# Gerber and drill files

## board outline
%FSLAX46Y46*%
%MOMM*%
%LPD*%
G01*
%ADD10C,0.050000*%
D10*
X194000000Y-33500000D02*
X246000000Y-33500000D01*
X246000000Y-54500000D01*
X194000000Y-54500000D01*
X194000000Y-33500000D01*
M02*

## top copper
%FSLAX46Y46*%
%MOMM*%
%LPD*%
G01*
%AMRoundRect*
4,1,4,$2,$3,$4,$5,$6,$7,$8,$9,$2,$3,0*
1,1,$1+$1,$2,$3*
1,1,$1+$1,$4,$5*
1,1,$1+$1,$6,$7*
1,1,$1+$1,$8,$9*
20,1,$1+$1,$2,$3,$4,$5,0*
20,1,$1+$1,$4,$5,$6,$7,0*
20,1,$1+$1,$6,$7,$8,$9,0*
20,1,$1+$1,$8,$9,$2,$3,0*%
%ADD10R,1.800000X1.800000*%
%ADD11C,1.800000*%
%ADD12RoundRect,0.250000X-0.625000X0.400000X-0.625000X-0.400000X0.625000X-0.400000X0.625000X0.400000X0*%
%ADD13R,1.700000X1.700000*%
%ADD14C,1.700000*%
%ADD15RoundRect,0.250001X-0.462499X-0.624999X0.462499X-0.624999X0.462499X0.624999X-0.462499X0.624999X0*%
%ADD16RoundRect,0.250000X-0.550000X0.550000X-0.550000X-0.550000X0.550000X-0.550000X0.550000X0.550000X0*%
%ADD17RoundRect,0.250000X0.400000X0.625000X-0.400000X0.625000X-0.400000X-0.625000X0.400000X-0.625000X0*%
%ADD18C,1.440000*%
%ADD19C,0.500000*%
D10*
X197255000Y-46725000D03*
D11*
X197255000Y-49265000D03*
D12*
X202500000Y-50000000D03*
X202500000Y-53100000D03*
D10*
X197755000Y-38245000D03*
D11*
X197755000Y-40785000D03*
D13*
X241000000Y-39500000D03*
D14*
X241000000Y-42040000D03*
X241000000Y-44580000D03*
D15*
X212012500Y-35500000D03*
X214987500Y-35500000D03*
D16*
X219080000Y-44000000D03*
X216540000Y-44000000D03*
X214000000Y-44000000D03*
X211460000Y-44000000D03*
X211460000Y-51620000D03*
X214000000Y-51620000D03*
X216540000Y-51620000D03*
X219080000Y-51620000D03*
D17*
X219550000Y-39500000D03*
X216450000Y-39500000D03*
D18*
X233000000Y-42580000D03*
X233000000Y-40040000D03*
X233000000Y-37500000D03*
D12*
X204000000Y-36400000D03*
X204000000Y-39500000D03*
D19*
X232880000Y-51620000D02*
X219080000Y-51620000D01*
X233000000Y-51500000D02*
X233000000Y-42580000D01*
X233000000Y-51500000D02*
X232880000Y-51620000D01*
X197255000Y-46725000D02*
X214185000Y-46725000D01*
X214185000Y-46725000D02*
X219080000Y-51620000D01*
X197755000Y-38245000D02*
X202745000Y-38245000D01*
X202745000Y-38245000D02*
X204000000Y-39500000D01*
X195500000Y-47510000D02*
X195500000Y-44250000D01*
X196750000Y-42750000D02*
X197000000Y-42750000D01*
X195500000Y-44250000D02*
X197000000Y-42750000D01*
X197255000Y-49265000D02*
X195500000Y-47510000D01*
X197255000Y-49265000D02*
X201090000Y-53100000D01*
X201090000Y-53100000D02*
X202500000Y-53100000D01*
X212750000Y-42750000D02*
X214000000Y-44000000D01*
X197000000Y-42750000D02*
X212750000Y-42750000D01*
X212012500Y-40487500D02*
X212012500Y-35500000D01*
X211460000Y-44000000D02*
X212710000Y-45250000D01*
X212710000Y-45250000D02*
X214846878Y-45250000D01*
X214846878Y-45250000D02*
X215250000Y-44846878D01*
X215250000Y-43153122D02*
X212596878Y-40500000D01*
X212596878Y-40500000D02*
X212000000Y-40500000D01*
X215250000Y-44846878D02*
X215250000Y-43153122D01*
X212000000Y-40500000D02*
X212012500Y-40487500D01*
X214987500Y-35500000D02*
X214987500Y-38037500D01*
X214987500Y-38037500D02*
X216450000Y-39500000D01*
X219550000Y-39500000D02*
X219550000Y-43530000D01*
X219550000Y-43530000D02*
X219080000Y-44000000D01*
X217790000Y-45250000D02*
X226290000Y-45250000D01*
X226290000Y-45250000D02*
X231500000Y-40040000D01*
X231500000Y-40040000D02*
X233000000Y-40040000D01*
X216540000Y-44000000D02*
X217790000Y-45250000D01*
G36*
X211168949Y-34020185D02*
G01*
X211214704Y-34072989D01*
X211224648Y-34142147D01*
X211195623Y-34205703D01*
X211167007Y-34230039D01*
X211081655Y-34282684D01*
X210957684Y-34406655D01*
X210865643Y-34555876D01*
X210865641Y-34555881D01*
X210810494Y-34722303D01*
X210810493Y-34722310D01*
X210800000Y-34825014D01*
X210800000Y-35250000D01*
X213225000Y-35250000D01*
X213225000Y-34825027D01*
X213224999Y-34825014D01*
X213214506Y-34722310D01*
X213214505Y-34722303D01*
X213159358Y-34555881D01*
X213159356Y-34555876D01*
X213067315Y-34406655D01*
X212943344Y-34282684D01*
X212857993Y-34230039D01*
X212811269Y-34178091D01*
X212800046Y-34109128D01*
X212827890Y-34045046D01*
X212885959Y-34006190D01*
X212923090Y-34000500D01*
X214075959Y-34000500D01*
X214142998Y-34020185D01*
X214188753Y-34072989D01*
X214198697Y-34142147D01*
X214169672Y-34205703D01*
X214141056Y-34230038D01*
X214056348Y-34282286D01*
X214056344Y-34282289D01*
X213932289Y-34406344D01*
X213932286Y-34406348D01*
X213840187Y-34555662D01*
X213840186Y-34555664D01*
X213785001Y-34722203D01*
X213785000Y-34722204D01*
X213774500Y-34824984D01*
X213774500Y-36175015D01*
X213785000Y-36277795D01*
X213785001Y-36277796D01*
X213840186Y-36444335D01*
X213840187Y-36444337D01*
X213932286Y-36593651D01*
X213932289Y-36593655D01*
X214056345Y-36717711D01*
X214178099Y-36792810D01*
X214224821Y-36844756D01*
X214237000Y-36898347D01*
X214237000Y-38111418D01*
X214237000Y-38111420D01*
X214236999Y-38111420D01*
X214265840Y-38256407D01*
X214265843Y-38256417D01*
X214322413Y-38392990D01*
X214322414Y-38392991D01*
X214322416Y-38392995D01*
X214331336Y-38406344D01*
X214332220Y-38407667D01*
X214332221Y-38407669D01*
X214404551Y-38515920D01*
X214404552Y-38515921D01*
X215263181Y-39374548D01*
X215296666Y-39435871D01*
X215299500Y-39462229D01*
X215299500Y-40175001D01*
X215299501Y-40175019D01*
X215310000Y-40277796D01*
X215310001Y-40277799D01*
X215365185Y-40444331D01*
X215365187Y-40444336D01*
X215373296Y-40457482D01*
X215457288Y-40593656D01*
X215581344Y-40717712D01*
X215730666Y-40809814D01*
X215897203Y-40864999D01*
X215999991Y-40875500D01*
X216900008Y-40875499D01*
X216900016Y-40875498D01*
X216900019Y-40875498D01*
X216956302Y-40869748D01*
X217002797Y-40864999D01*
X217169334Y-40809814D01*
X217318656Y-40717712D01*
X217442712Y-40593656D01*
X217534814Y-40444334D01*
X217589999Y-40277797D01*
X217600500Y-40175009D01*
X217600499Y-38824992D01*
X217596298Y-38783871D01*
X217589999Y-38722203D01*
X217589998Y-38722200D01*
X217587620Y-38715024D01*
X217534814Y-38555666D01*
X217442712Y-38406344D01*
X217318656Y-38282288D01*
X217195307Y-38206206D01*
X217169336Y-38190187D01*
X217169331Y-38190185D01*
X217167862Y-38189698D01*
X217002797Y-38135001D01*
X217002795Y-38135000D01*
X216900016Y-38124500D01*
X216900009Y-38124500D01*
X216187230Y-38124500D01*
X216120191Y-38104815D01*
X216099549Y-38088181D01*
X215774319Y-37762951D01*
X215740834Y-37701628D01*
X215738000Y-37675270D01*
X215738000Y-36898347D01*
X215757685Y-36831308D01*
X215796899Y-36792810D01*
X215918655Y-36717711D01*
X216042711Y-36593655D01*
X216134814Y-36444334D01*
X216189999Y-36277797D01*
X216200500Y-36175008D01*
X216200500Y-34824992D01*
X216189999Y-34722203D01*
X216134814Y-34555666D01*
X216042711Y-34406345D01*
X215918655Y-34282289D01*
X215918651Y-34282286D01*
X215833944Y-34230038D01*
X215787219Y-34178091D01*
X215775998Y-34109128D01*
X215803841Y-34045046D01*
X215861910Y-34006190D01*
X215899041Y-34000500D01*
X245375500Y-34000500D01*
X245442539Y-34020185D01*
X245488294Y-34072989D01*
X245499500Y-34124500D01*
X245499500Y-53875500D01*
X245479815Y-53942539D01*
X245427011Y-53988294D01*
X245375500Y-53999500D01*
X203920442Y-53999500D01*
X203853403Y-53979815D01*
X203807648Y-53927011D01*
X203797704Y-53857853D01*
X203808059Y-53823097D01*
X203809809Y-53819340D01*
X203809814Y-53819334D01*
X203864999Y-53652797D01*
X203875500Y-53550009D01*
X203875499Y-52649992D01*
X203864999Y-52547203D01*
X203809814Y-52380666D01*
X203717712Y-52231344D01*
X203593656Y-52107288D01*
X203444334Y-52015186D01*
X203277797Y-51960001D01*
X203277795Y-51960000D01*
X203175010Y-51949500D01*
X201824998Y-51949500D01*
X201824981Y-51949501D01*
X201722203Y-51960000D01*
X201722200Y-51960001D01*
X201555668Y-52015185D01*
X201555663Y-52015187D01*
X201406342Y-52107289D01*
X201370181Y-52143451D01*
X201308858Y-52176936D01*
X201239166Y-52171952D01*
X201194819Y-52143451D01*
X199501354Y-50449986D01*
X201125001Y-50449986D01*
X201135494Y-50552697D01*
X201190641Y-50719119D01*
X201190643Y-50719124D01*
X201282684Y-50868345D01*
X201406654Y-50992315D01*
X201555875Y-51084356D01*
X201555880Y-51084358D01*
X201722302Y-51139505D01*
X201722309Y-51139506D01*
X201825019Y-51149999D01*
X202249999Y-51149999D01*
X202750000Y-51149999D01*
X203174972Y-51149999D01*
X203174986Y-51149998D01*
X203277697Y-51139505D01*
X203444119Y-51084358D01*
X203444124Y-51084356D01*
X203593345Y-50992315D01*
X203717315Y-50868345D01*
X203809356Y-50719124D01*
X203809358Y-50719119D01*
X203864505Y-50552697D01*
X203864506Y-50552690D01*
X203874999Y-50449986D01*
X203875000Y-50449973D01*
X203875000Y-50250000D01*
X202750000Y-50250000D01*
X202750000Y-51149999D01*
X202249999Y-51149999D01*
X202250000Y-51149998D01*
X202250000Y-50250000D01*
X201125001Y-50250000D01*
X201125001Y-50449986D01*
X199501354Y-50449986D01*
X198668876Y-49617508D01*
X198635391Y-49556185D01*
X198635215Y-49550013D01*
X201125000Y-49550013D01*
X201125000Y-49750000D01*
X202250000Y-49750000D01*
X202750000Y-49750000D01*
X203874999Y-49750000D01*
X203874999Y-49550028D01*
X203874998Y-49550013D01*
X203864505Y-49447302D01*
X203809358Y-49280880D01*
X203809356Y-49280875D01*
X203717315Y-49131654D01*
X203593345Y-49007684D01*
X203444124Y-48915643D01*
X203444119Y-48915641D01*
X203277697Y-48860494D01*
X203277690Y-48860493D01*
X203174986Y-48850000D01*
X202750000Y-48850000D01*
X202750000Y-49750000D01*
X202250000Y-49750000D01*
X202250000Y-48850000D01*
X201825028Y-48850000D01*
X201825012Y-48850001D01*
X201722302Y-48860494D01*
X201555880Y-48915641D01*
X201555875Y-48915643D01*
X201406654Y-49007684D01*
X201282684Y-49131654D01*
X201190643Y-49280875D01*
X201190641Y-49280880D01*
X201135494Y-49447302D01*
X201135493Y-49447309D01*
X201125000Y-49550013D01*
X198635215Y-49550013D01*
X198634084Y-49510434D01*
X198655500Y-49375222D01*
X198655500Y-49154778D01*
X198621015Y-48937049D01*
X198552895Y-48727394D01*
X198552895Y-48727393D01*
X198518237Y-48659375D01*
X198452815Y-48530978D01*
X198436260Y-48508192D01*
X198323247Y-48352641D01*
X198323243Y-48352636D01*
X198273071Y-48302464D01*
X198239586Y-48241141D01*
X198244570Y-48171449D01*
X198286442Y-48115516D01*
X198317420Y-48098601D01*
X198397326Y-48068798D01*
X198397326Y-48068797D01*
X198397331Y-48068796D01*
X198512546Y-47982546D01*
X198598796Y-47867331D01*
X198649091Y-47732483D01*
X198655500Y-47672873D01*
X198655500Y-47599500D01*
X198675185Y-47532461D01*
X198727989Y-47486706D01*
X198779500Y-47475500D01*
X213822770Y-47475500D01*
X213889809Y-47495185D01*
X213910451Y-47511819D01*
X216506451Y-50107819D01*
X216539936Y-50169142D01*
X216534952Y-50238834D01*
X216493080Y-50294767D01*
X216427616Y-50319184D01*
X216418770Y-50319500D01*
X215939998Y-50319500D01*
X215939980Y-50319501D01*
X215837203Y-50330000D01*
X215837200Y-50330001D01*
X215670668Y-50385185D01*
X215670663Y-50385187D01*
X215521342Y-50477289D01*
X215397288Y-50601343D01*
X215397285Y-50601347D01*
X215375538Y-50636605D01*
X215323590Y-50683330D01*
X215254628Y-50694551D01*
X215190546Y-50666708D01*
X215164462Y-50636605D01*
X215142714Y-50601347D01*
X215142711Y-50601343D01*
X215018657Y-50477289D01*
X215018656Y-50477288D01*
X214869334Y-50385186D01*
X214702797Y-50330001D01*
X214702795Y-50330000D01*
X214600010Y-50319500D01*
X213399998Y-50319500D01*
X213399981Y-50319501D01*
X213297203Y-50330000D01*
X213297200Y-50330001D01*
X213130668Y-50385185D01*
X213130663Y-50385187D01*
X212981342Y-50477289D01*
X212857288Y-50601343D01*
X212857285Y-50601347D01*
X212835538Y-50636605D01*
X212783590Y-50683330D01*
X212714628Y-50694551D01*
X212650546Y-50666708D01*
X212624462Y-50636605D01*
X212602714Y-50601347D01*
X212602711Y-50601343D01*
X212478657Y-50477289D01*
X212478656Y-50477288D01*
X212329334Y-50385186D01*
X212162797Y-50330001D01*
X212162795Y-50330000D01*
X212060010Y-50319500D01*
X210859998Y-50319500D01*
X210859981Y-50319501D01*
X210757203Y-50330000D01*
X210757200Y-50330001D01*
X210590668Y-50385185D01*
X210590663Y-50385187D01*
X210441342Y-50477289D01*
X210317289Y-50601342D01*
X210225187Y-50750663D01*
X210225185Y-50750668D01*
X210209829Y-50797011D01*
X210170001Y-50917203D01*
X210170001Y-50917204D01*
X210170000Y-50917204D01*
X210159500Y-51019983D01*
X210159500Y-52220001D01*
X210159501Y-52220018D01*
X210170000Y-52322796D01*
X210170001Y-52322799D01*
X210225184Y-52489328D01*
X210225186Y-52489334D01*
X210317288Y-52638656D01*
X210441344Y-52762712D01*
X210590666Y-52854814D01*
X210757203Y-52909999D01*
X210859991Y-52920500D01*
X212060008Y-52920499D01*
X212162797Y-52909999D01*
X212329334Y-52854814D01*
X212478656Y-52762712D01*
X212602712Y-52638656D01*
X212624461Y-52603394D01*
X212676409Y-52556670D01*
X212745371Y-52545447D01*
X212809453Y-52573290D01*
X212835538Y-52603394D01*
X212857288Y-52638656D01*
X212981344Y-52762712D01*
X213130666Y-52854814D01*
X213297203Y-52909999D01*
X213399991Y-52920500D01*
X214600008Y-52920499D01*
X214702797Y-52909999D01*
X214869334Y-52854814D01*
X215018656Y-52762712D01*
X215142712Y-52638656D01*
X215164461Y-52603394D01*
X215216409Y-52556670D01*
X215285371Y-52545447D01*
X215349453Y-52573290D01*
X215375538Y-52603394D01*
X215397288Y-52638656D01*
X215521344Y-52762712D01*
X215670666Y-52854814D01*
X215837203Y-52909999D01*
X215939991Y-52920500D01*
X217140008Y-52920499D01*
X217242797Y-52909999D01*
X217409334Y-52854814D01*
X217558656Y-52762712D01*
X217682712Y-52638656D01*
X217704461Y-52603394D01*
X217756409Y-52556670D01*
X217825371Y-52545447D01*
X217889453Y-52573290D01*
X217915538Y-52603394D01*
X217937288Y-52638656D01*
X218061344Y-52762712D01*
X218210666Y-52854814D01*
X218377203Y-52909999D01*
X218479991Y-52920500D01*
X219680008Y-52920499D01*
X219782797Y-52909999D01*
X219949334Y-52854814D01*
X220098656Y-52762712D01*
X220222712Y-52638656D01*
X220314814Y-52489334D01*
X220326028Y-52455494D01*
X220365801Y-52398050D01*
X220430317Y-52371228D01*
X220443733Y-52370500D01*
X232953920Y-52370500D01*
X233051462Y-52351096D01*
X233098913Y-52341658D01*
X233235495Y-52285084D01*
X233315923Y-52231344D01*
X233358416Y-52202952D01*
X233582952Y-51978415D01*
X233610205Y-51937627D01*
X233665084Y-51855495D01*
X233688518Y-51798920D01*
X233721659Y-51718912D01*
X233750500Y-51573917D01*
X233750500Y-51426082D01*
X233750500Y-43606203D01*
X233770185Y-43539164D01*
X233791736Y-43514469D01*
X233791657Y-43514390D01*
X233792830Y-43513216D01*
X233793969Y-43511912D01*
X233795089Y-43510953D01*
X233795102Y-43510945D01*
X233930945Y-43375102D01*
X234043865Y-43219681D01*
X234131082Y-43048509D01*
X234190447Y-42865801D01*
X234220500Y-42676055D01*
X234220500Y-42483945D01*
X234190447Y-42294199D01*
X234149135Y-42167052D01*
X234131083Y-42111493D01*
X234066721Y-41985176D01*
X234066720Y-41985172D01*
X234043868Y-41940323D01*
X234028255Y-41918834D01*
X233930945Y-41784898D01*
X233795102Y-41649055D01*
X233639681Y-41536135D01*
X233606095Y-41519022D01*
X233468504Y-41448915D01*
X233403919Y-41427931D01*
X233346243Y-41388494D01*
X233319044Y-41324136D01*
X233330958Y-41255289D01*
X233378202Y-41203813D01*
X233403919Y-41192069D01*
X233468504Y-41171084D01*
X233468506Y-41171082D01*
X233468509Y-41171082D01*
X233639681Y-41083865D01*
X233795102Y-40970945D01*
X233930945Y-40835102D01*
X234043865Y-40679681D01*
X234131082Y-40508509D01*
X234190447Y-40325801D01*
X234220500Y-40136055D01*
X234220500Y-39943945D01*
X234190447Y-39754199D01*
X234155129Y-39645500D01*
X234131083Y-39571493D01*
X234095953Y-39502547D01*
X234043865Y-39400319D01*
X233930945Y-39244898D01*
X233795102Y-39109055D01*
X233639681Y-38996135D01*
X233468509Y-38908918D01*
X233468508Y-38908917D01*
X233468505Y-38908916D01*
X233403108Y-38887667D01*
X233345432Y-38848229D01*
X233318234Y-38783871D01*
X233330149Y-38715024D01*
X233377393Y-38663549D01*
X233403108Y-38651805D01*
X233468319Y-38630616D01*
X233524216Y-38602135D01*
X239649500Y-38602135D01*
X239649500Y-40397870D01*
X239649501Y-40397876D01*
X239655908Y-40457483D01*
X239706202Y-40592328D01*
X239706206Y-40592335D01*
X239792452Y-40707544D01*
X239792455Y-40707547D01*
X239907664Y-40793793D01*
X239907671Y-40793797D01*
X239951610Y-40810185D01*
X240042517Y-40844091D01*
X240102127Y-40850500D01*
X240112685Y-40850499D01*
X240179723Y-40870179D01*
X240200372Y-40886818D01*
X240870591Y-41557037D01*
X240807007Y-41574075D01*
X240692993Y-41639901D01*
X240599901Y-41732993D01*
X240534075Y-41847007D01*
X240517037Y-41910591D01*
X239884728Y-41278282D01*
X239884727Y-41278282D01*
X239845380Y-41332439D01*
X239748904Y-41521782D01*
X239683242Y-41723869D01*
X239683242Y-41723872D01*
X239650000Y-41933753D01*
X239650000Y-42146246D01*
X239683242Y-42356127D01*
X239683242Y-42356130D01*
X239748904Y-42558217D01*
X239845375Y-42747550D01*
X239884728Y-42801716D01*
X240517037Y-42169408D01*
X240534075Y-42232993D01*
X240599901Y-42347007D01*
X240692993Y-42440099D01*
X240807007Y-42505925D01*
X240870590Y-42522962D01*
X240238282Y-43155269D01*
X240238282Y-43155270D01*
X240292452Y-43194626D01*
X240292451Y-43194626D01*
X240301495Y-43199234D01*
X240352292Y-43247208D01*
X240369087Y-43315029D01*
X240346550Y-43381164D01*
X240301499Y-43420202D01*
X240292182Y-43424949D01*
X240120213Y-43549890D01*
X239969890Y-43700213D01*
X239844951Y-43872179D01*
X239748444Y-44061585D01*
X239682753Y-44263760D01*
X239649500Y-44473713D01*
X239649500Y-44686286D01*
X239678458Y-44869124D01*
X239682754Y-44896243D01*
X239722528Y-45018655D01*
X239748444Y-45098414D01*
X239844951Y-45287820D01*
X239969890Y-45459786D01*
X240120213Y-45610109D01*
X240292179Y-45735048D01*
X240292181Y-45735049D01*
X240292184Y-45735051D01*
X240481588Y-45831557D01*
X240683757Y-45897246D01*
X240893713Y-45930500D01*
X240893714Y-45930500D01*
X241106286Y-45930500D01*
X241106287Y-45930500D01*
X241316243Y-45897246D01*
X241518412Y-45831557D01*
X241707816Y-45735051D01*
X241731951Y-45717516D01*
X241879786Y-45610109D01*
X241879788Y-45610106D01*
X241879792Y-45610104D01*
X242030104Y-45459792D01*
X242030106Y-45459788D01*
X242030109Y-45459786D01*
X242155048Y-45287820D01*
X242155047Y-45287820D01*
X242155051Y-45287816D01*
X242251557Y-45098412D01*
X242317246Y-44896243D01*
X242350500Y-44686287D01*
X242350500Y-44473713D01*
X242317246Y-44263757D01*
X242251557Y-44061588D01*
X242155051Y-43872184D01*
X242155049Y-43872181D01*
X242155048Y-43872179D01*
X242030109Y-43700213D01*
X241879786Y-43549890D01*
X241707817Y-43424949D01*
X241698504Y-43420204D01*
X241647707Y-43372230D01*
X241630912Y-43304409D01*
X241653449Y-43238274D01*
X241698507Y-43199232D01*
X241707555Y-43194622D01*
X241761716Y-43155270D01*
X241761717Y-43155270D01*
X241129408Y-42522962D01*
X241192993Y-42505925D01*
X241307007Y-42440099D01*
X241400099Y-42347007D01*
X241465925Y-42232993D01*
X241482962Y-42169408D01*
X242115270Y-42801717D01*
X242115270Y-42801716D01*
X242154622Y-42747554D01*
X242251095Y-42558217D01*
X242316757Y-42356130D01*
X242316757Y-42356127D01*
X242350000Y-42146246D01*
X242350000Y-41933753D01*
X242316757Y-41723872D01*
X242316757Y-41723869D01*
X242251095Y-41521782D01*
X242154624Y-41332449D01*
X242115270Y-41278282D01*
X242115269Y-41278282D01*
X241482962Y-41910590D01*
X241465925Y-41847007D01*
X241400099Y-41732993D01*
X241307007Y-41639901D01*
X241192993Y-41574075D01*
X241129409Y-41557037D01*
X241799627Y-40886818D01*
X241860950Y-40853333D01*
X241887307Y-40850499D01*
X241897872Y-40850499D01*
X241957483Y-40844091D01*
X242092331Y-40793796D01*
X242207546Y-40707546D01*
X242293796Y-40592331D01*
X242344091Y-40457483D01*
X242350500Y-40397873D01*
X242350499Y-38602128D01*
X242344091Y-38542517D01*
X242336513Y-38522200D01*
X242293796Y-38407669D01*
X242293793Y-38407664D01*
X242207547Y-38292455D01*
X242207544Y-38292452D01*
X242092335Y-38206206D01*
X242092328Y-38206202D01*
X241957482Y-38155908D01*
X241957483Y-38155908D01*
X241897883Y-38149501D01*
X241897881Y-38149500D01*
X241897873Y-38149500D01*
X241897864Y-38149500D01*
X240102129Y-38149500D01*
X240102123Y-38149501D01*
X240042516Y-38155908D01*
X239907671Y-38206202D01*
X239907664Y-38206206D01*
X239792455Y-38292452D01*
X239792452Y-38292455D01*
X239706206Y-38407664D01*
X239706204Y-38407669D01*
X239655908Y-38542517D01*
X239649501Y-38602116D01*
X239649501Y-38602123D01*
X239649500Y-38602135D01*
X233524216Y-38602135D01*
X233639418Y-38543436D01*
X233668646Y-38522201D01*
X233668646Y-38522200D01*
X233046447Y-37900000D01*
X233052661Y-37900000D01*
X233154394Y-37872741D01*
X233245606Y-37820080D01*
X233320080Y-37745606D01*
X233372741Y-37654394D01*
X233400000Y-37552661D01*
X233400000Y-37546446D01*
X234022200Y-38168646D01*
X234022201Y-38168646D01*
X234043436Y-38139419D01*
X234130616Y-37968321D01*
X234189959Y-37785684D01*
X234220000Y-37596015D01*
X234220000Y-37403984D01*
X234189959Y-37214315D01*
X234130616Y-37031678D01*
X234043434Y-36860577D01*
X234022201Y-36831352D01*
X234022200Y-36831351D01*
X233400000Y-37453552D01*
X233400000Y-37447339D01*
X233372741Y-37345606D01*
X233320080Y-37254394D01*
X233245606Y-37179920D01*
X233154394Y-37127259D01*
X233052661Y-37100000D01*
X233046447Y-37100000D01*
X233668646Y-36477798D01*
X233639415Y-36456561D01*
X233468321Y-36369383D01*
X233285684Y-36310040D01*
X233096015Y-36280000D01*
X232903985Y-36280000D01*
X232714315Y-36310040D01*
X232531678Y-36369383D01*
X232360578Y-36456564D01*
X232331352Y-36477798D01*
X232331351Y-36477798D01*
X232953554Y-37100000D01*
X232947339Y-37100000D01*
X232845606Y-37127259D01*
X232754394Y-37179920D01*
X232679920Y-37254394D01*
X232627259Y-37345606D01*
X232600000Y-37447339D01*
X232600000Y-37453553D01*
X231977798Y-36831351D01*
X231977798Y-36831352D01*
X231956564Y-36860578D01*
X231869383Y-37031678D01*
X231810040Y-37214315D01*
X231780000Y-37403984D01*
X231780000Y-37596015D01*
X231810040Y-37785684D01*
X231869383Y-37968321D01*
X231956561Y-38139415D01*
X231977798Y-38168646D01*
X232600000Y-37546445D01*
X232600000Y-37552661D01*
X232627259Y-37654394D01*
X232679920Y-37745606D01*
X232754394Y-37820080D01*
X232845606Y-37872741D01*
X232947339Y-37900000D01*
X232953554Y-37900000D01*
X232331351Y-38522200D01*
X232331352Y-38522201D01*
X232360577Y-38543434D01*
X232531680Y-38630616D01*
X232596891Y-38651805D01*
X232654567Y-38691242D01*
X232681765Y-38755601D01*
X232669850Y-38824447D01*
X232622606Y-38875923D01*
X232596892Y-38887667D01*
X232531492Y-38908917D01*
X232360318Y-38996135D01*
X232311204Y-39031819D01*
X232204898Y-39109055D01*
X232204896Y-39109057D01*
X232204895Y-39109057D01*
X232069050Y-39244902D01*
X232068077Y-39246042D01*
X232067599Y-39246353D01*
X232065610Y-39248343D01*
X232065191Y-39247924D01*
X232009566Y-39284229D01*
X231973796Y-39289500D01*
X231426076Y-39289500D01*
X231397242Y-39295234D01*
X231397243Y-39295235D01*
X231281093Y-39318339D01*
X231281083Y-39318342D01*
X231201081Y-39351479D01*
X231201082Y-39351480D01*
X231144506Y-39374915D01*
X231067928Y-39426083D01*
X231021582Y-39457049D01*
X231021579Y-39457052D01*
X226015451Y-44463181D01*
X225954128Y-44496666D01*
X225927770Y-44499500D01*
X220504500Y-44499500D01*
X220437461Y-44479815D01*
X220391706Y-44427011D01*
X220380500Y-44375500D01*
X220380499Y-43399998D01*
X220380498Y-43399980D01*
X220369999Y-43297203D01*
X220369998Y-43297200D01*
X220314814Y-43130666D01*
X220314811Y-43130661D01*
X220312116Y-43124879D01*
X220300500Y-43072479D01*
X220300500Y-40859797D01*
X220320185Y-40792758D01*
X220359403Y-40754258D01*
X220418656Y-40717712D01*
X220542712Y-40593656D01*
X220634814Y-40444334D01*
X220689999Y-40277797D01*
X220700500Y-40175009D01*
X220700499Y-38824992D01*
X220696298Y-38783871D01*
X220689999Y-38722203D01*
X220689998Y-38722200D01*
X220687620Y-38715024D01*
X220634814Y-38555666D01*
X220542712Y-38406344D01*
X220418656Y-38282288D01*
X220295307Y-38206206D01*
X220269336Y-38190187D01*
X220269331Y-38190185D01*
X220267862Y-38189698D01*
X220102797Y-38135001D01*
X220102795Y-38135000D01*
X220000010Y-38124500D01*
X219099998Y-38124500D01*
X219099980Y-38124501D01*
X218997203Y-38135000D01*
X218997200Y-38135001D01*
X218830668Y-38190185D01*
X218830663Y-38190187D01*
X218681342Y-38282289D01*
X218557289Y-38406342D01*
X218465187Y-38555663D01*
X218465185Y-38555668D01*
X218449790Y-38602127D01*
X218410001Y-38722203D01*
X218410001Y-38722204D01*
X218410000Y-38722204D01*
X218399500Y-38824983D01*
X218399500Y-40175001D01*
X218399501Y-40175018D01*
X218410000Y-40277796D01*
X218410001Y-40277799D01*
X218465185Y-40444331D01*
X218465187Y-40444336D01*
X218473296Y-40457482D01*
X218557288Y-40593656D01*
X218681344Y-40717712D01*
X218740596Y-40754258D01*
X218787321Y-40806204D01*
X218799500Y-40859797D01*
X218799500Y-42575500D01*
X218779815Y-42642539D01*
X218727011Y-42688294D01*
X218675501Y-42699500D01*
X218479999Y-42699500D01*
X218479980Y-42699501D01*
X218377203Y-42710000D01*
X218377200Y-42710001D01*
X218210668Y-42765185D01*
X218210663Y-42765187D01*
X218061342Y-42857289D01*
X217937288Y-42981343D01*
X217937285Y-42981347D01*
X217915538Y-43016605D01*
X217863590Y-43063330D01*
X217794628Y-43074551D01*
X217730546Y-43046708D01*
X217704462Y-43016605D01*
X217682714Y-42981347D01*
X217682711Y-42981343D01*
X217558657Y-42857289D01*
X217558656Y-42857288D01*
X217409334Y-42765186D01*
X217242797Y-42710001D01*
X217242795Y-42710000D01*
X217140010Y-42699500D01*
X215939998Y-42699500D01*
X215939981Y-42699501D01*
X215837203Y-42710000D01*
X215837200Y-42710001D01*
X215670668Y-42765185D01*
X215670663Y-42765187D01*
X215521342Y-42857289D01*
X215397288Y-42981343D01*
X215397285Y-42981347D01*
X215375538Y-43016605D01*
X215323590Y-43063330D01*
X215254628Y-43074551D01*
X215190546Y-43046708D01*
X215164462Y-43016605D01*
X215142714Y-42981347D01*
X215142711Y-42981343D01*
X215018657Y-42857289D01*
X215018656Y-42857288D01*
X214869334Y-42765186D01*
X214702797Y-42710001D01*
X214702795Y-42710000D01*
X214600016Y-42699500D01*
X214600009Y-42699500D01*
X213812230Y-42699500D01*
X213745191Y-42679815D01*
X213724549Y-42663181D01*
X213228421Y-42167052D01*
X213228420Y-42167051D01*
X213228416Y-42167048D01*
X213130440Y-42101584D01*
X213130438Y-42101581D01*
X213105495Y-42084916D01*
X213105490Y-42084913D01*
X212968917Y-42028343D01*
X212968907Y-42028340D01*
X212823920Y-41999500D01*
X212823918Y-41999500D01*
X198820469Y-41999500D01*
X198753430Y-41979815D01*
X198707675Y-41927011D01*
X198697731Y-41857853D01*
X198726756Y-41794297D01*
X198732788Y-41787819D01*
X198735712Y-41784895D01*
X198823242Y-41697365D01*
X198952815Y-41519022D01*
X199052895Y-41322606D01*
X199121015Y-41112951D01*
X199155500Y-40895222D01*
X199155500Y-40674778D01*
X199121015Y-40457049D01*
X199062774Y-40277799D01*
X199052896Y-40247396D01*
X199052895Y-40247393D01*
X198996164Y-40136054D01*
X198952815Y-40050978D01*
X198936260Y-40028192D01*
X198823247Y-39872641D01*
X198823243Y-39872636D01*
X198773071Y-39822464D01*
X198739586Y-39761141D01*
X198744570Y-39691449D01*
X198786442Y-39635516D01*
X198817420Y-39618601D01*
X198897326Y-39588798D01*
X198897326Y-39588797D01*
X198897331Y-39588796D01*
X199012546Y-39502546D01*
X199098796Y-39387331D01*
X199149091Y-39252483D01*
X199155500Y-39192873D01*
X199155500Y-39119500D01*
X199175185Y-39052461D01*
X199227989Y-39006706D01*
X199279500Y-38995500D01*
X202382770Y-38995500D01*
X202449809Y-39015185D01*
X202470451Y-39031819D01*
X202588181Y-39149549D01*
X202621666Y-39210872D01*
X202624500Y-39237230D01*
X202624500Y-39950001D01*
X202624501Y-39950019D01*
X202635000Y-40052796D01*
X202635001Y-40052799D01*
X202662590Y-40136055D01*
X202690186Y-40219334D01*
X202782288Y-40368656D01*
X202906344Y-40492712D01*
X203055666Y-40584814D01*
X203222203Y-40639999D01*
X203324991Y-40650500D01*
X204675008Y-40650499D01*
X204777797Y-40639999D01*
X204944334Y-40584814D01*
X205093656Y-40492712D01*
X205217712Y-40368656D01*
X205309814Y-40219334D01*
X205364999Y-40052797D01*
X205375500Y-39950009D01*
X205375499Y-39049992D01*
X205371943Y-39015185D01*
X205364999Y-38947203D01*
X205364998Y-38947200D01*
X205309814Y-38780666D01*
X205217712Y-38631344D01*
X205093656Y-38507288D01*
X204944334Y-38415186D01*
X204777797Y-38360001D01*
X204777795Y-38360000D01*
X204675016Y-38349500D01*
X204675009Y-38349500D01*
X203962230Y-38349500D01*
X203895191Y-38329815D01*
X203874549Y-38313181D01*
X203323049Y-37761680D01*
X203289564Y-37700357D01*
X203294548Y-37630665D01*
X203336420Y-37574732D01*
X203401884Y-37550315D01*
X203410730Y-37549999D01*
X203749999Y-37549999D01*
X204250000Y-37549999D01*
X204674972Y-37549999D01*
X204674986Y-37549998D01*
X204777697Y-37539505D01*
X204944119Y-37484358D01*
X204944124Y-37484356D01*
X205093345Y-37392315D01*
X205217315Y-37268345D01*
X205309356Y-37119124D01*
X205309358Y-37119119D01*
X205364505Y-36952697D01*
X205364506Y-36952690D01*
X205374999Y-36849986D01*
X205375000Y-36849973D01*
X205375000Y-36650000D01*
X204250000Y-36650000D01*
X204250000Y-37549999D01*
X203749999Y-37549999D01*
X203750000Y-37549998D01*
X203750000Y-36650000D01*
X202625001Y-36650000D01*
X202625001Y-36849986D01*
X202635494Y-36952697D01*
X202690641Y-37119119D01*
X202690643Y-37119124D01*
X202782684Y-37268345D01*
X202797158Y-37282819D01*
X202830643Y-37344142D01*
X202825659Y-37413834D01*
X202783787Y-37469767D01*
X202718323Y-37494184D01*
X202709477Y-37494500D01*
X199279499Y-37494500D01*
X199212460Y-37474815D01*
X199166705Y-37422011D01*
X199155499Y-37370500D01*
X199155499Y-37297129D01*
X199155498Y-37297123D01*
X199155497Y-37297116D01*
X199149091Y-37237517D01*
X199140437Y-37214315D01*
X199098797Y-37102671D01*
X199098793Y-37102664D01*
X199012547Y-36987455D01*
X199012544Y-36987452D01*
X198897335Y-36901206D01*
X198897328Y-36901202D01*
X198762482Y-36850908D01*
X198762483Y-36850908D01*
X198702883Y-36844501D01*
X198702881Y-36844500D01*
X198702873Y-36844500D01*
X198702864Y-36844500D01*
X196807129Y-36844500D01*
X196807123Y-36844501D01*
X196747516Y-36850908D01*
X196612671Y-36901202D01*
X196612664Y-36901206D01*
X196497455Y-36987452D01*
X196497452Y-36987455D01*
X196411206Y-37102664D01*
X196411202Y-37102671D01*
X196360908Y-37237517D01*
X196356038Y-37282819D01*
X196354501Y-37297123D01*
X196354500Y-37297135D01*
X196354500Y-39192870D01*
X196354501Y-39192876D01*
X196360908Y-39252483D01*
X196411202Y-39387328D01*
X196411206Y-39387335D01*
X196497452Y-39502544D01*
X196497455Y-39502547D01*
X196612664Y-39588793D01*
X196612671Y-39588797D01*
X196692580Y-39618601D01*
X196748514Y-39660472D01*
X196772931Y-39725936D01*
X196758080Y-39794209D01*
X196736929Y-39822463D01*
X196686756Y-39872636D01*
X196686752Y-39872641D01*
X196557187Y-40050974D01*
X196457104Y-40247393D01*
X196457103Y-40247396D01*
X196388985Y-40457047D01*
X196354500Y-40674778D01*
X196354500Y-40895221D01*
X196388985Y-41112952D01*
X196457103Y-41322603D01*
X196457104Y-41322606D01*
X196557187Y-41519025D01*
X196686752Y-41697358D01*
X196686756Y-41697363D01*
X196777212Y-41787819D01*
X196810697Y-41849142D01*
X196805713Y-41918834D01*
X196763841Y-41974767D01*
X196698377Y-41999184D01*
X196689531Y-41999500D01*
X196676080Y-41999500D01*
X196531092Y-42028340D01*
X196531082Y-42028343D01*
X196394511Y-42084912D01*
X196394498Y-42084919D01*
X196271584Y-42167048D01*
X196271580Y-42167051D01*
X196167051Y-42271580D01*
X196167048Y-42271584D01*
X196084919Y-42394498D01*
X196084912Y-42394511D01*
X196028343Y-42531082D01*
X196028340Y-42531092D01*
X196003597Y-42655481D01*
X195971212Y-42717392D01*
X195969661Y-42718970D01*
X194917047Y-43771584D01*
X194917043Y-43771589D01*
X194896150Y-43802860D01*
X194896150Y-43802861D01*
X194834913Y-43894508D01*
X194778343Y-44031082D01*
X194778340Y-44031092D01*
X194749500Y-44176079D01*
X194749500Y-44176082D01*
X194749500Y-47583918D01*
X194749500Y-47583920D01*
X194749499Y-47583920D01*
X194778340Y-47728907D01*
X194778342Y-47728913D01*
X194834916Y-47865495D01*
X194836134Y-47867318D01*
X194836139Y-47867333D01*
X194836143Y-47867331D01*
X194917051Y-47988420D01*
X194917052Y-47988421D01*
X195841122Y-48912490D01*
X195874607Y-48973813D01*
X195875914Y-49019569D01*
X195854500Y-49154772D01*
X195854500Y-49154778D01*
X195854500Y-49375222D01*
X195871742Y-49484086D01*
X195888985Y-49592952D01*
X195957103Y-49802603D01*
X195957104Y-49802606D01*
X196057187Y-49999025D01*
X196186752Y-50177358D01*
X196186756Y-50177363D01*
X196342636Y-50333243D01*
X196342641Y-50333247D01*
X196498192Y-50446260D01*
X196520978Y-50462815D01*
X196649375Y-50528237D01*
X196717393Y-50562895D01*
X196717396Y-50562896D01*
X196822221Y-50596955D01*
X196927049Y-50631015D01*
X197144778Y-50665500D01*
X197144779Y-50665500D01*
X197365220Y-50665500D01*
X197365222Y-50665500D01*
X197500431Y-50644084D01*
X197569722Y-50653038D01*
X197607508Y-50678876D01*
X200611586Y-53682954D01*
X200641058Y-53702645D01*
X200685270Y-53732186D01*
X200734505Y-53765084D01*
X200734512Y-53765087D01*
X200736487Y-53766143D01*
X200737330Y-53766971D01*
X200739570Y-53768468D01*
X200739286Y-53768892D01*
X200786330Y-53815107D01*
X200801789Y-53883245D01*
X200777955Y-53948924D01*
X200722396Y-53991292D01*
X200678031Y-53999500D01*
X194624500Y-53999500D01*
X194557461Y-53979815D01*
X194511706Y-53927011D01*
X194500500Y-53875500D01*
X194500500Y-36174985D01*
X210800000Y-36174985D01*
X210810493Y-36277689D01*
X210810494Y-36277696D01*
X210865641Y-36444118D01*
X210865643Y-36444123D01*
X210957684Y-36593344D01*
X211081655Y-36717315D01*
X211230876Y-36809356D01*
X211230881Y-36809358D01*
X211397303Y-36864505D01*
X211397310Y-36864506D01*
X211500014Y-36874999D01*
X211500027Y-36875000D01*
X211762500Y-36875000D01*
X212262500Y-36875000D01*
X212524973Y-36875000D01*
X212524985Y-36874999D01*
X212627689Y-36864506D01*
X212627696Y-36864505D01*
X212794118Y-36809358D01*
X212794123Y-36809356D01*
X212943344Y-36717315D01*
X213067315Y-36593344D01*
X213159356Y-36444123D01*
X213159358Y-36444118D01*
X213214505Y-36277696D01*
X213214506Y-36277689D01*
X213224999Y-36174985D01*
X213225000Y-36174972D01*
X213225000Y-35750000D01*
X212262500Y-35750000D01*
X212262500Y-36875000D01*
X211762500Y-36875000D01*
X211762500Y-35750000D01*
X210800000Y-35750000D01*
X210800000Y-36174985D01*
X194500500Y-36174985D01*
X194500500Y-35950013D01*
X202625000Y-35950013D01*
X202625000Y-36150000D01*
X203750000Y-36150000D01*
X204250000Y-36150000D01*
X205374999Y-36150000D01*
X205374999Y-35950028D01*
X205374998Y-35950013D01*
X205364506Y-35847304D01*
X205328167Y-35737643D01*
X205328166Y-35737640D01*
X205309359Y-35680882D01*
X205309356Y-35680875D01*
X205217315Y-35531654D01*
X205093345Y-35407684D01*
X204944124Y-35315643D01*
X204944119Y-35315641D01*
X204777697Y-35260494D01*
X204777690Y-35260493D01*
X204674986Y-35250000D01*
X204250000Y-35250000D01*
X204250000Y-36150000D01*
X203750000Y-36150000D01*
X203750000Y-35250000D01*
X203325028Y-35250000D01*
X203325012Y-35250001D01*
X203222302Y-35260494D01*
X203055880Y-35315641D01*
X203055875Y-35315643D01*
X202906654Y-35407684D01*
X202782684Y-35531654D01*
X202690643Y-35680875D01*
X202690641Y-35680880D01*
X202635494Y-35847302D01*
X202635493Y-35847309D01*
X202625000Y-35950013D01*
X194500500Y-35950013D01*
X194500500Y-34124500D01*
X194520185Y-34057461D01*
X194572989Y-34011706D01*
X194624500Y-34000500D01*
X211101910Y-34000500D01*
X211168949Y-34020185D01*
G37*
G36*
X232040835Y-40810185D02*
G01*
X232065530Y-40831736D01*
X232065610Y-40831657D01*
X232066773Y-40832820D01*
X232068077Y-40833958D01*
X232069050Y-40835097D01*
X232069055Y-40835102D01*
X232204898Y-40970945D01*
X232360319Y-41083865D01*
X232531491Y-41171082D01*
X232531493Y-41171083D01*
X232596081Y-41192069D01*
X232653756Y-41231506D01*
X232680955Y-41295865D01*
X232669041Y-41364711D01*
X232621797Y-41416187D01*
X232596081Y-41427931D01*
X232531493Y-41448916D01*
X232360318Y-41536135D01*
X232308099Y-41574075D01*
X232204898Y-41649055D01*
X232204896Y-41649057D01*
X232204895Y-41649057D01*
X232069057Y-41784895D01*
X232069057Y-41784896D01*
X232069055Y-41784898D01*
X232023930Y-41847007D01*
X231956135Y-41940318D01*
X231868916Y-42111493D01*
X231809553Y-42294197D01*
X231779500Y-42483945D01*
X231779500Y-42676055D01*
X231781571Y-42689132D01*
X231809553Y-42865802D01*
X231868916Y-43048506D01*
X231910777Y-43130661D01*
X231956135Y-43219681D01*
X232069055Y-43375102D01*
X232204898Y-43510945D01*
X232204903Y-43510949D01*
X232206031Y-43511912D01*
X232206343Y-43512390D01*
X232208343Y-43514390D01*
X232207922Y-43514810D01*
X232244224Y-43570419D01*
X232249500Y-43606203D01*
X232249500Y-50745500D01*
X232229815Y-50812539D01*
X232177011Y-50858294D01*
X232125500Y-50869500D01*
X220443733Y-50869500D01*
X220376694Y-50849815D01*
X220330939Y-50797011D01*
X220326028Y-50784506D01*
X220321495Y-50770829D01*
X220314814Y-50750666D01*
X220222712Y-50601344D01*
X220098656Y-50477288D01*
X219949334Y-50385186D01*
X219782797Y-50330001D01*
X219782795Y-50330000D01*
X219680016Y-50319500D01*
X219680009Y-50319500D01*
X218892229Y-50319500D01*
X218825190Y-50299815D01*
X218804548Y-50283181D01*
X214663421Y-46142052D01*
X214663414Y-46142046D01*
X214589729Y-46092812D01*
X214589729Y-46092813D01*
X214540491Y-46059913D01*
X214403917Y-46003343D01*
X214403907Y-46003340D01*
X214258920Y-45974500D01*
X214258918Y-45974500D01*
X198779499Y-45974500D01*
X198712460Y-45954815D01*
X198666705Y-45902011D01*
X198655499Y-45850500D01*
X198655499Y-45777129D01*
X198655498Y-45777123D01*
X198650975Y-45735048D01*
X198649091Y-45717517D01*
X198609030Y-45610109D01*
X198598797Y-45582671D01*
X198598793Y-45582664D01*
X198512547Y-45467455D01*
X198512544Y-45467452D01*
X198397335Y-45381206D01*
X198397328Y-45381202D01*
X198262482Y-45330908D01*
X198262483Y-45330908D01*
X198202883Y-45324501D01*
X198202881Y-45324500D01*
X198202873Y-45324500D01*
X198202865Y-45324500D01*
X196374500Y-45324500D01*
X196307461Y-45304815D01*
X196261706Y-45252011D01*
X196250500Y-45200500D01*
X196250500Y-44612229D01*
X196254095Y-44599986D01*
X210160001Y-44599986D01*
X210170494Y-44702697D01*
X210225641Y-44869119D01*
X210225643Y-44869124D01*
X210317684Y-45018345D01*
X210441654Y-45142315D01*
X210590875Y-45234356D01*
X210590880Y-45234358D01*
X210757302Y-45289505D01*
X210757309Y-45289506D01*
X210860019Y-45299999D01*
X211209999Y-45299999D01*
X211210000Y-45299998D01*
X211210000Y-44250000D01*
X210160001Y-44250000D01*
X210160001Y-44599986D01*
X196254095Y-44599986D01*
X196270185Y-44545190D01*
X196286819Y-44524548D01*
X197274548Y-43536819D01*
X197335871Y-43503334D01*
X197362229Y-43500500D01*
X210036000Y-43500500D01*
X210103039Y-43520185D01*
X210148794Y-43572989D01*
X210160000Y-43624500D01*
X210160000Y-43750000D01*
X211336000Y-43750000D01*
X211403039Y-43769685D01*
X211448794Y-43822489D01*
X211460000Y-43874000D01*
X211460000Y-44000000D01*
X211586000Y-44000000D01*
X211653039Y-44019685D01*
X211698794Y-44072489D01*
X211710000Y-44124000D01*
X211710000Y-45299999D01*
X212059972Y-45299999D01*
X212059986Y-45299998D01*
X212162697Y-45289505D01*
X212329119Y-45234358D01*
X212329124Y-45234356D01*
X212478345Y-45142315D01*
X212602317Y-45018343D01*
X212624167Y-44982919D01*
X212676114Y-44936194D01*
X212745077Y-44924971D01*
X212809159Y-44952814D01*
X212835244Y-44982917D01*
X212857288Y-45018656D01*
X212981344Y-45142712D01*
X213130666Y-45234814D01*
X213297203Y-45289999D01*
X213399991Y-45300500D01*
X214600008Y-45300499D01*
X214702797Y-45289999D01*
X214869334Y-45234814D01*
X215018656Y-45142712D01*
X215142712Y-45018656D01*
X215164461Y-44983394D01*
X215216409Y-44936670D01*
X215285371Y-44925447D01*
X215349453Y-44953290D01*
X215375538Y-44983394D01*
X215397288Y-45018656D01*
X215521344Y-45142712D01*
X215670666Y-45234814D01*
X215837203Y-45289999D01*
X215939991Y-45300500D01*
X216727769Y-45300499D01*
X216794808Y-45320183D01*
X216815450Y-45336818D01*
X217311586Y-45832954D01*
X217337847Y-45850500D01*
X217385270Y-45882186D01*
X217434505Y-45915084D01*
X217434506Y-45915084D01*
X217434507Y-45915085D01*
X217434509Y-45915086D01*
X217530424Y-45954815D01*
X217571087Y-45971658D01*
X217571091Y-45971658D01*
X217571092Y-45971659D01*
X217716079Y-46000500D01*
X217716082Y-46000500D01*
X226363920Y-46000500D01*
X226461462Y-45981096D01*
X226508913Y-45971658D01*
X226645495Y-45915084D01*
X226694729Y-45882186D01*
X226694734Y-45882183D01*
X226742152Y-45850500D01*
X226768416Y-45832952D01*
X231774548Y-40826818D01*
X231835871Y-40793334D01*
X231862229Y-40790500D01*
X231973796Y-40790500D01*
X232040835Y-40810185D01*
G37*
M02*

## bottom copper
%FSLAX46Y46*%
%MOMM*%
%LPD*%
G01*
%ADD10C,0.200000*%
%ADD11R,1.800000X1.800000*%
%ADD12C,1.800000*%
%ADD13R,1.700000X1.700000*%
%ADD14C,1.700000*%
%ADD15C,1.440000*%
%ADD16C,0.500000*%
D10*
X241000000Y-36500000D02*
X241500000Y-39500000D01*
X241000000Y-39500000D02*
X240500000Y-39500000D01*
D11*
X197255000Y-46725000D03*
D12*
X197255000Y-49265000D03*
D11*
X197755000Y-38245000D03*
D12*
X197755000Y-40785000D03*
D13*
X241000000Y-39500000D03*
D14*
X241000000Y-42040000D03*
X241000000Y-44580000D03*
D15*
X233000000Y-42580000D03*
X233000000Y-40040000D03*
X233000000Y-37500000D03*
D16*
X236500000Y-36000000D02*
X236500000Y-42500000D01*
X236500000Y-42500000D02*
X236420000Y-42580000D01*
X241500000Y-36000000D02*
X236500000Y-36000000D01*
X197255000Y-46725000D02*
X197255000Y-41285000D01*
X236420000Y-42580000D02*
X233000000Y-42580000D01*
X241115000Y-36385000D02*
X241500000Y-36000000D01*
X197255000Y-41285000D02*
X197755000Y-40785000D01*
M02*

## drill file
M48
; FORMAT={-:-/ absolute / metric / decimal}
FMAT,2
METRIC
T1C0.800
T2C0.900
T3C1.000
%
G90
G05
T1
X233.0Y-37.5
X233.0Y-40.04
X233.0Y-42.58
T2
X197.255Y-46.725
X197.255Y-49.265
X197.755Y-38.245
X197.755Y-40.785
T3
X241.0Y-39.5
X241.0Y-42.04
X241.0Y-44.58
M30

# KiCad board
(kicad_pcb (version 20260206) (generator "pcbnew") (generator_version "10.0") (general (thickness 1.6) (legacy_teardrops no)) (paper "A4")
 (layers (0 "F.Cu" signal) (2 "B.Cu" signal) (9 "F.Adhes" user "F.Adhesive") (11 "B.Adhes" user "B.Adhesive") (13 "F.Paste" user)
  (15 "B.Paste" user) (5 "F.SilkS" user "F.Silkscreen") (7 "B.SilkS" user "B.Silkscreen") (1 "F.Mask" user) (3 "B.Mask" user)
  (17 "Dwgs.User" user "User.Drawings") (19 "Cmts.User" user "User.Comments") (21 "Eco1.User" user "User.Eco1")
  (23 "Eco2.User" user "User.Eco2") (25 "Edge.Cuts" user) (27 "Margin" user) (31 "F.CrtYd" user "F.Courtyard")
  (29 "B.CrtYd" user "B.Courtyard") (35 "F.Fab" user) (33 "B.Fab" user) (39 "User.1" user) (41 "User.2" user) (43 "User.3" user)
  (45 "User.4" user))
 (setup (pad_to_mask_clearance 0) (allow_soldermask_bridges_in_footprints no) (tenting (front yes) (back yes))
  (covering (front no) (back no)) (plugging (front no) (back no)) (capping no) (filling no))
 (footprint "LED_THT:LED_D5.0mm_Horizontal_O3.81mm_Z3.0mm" (layer "F.Cu") (at 197.255 46.725 -90)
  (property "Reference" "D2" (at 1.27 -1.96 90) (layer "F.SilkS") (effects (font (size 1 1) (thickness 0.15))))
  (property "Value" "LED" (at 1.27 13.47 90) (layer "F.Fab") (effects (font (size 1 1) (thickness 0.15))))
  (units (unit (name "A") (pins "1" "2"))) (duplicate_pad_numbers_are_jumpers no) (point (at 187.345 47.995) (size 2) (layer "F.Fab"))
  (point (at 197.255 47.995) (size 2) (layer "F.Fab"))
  (pad "1" thru_hole rect (at 0 0 270) (size 1.8 1.8) (drill 0.9) (layers "*.Cu" "*.Mask") (remove_unused_layers no) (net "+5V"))
  (pad "2" thru_hole circle (at 2.54 0 270) (size 1.8 1.8) (drill 0.9) (layers "*.Cu" "*.Mask") (remove_unused_layers no) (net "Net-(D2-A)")))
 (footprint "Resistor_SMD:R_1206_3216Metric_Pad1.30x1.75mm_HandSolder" (layer "F.Cu") (at 202.5 51.55 -90)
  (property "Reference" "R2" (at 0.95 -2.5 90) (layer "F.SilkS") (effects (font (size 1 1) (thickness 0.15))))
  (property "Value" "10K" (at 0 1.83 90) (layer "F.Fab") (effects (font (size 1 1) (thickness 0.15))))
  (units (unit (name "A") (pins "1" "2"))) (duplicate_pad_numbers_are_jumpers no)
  (pad "1" smd roundrect (at -1.55 0 270) (size 1.3 1.75) (layers "F.Cu" "F.Mask" "F.Paste") (roundrect_rratio 0.192308) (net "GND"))
  (pad "2" smd roundrect (at 1.55 0 270) (size 1.3 1.75) (layers "F.Cu" "F.Mask" "F.Paste") (roundrect_rratio 0.192308) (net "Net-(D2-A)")))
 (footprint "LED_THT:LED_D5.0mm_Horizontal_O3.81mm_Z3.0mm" (layer "F.Cu") (at 197.755 38.245 -90)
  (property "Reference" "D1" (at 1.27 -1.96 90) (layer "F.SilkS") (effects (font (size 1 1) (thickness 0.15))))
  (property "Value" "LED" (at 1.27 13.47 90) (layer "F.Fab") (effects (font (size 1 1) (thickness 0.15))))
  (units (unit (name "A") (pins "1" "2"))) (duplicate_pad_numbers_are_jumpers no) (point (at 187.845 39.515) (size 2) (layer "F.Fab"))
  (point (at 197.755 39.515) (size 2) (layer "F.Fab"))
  (pad "1" thru_hole rect (at 0 0 270) (size 1.8 1.8) (drill 0.9) (layers "*.Cu" "*.Mask") (remove_unused_layers no) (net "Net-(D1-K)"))
  (pad "2" thru_hole circle (at 2.54 0 270) (size 1.8 1.8) (drill 0.9) (layers "*.Cu" "*.Mask") (remove_unused_layers no) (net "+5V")))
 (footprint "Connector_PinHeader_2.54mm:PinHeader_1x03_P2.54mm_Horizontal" (layer "F.Cu") (at 241 39.5)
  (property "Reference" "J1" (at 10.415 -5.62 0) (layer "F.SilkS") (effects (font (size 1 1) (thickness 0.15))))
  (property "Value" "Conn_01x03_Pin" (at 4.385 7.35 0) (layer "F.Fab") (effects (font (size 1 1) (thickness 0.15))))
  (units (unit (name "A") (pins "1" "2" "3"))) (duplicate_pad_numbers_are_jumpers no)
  (pad "1" thru_hole rect (at 0 0) (size 1.7 1.7) (drill 1) (layers "*.Cu" "*.Mask") (remove_unused_layers no) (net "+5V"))
  (pad "2" thru_hole circle (at 0 2.54) (size 1.7 1.7) (drill 1) (layers "*.Cu" "*.Mask") (remove_unused_layers no) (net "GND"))
  (pad "3" thru_hole circle (at 0 5.08) (size 1.7 1.7) (drill 1) (layers "*.Cu" "*.Mask") (remove_unused_layers no) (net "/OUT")))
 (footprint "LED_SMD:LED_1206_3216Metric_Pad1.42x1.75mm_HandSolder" (layer "F.Cu") (at 213.5 35.5)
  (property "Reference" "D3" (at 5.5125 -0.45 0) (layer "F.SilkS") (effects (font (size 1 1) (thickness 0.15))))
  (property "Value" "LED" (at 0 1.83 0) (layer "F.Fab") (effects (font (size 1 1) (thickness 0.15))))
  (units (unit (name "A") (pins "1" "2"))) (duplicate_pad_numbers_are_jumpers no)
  (pad "1" smd roundrect (at -1.4875 0) (size 1.425 1.75) (layers "F.Cu" "F.Mask" "F.Paste") (roundrect_rratio 0.175439) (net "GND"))
  (pad "2" smd roundrect (at 1.4875 0) (size 1.425 1.75) (layers "F.Cu" "F.Mask" "F.Paste") (roundrect_rratio 0.175439) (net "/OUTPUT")))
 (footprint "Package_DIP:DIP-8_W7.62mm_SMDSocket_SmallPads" (layer "F.Cu") (at 215.27 47.81 -90)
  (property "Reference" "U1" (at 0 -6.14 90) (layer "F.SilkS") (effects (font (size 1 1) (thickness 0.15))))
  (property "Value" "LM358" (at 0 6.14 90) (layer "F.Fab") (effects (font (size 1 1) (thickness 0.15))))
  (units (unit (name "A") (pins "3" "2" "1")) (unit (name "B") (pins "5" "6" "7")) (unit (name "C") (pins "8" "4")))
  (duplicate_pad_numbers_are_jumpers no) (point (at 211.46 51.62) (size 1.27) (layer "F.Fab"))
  (pad "1" smd roundrect (at -3.81 -3.81 270) (size 1.6 1.6) (layers "F.Cu" "F.Mask" "F.Paste") (roundrect_rratio 0.15625)
   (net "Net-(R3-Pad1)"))
  (pad "2" smd roundrect (at -3.81 -1.27 270) (size 1.6 1.6) (layers "F.Cu" "F.Mask" "F.Paste") (roundrect_rratio 0.15625)
   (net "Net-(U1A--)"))
  (pad "3" smd roundrect (at -3.81 1.27 270) (size 1.6 1.6) (layers "F.Cu" "F.Mask" "F.Paste") (roundrect_rratio 0.15625) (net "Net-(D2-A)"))
  (pad "4" smd roundrect (at -3.81 3.81 270) (size 1.6 1.6) (layers "F.Cu" "F.Mask" "F.Paste") (roundrect_rratio 0.15625) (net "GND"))
  (pad "5" smd roundrect (at 3.81 3.81 270) (size 1.6 1.6) (layers "F.Cu" "F.Mask" "F.Paste") (roundrect_rratio 0.15625))
  (pad "6" smd roundrect (at 3.81 1.27 270) (size 1.6 1.6) (layers "F.Cu" "F.Mask" "F.Paste") (roundrect_rratio 0.15625))
  (pad "7" smd roundrect (at 3.81 -1.27 270) (size 1.6 1.6) (layers "F.Cu" "F.Mask" "F.Paste") (roundrect_rratio 0.15625))
  (pad "8" smd roundrect (at 3.81 -3.81 270) (size 1.6 1.6) (layers "F.Cu" "F.Mask" "F.Paste") (roundrect_rratio 0.15625) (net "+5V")))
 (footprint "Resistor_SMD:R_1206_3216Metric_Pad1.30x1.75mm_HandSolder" (layer "F.Cu") (at 218 39.5 180)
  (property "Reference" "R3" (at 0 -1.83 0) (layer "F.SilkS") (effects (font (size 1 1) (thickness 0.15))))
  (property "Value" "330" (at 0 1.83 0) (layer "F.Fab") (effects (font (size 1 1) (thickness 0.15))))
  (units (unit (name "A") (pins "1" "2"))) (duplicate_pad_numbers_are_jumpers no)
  (pad "1" smd roundrect (at -1.55 0 180) (size 1.3 1.75) (layers "F.Cu" "F.Mask" "F.Paste") (roundrect_rratio 0.192308)
   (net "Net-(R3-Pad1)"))
  (pad "2" smd roundrect (at 1.55 0 180) (size 1.3 1.75) (layers "F.Cu" "F.Mask" "F.Paste") (roundrect_rratio 0.192308) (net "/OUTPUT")))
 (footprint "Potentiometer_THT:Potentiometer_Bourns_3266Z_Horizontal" (layer "F.Cu") (at 233 42.58 -90)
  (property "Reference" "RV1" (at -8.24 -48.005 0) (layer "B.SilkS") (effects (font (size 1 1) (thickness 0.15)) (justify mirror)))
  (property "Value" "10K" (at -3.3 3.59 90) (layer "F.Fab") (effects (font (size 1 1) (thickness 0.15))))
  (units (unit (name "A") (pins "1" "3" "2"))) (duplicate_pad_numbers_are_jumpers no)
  (pad "1" thru_hole circle (at 0 0 270) (size 1.44 1.44) (drill 0.8) (layers "*.Cu" "*.Mask") (remove_unused_layers no) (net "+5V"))
  (pad "2" thru_hole circle (at -2.54 0 270) (size 1.44 1.44) (drill 0.8) (layers "*.Cu" "*.Mask") (remove_unused_layers no)
   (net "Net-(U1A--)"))
  (pad "3" thru_hole circle (at -5.08 0 270) (size 1.44 1.44) (drill 0.8) (layers "*.Cu" "*.Mask") (remove_unused_layers no) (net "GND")))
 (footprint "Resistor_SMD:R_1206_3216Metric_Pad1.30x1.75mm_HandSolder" (layer "F.Cu") (at 204 37.95 -90)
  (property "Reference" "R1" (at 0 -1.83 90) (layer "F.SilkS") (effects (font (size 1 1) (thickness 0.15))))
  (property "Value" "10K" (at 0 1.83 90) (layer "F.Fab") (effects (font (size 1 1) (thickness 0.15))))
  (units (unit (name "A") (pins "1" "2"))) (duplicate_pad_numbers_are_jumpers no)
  (pad "1" smd roundrect (at -1.55 0 270) (size 1.3 1.75) (layers "F.Cu" "F.Mask" "F.Paste") (roundrect_rratio 0.192308) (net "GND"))
  (pad "2" smd roundrect (at 1.55 0 270) (size 1.3 1.75) (layers "F.Cu" "F.Mask" "F.Paste") (roundrect_rratio 0.192308) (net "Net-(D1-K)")))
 (gr_line (start 241 36.5) (end 241.5 39.5) (stroke (width 0.2) (type default)) (layer "B.Cu") (net "+5V"))
 (gr_line (start 241 39.5) (end 240.5 39.5) (stroke (width 0.2) (type default)) (layer "B.Cu") (net "+5V"))
 (gr_rect (start 194 33.5) (end 246 54.5) (stroke (width 0.05) (type default)) (fill no) (layer "Edge.Cuts"))
 (segment (start 232.88 51.62) (end 219.08 51.62) (width 0.5) (layer "F.Cu") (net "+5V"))
 (segment (start 233 51.5) (end 233 42.58) (width 0.5) (layer "F.Cu") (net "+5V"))
 (segment (start 233 51.5) (end 232.88 51.62) (width 0.5) (layer "F.Cu") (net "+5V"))
 (segment (start 197.255 46.725) (end 214.185 46.725) (width 0.5) (layer "F.Cu") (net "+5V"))
 (segment (start 214.185 46.725) (end 219.08 51.62) (width 0.5) (layer "F.Cu") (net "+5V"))
 (segment (start 236.5 36) (end 236.5 42.5) (width 0.5) (layer "B.Cu") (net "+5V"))
 (segment (start 236.5 42.5) (end 236.42 42.58) (width 0.5) (layer "B.Cu") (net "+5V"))
 (segment (start 241.5 36) (end 236.5 36) (width 0.5) (layer "B.Cu") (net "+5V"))
 (segment (start 197.255 46.725) (end 197.255 41.285) (width 0.5) (layer "B.Cu") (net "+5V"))
 (segment (start 236.42 42.58) (end 233 42.58) (width 0.5) (layer "B.Cu") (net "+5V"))
 (segment (start 241.115 36.385) (end 241.5 36) (width 0.5) (layer "B.Cu") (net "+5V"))
 (segment (start 197.255 41.285) (end 197.755 40.785) (width 0.5) (layer "B.Cu") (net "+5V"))
 (segment (start 197.755 38.245) (end 202.745 38.245) (width 0.5) (layer "F.Cu") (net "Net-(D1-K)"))
 (segment (start 202.745 38.245) (end 204 39.5) (width 0.5) (layer "F.Cu") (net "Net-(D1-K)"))
 (segment (start 195.5 47.51) (end 195.5 44.25) (width 0.5) (layer "F.Cu") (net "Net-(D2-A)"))
 (segment (start 196.75 42.75) (end 197 42.75) (width 0.5) (layer "F.Cu") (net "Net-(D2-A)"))
 (segment (start 195.5 44.25) (end 197 42.75) (width 0.5) (layer "F.Cu") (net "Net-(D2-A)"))
 (segment (start 197.255 49.265) (end 195.5 47.51) (width 0.5) (layer "F.Cu") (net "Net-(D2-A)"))
 (segment (start 197.255 49.265) (end 201.09 53.1) (width 0.5) (layer "F.Cu") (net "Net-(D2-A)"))
 (segment (start 201.09 53.1) (end 202.5 53.1) (width 0.5) (layer "F.Cu") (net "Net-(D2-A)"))
 (segment (start 212.75 42.75) (end 214 44) (width 0.5) (layer "F.Cu") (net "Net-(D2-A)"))
 (segment (start 197 42.75) (end 212.75 42.75) (width 0.5) (layer "F.Cu") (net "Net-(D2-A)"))
 (segment (start 212.0125 40.4875) (end 212.0125 35.5) (width 0.5) (layer "F.Cu") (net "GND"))
 (segment (start 211.46 44) (end 212.71 45.25) (width 0.5) (layer "F.Cu") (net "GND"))
 (segment (start 212.71 45.25) (end 214.846878 45.25) (width 0.5) (layer "F.Cu") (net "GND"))
 (segment (start 214.846878 45.25) (end 215.25 44.846878) (width 0.5) (layer "F.Cu") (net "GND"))
 (segment (start 215.25 43.153122) (end 212.596878 40.5) (width 0.5) (layer "F.Cu") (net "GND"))
 (segment (start 212.596878 40.5) (end 212 40.5) (width 0.5) (layer "F.Cu") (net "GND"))
 (segment (start 215.25 44.846878) (end 215.25 43.153122) (width 0.5) (layer "F.Cu") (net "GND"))
 (segment (start 212 40.5) (end 212.0125 40.4875) (width 0.5) (layer "F.Cu") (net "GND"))
 (segment (start 214.9875 35.5) (end 214.9875 38.0375) (width 0.5) (layer "F.Cu") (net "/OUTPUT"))
 (segment (start 214.9875 38.0375) (end 216.45 39.5) (width 0.5) (layer "F.Cu") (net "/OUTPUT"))
 (segment (start 219.55 39.5) (end 219.55 43.53) (width 0.5) (layer "F.Cu") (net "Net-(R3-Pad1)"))
 (segment (start 219.55 43.53) (end 219.08 44) (width 0.5) (layer "F.Cu") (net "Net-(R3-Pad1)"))
 (segment (start 217.79 45.25) (end 226.29 45.25) (width 0.5) (layer "F.Cu") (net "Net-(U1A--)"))
 (segment (start 226.29 45.25) (end 231.5 40.04) (width 0.5) (layer "F.Cu") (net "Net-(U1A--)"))
 (segment (start 231.5 40.04) (end 233 40.04) (width 0.5) (layer "F.Cu") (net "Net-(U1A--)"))
 (segment (start 216.54 44) (end 217.79 45.25) (width 0.5) (layer "F.Cu") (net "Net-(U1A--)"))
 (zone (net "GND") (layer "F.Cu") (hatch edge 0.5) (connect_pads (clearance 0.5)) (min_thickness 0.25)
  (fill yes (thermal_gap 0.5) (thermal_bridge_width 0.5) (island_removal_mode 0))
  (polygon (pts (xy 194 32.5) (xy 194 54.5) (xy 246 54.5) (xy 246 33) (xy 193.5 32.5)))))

